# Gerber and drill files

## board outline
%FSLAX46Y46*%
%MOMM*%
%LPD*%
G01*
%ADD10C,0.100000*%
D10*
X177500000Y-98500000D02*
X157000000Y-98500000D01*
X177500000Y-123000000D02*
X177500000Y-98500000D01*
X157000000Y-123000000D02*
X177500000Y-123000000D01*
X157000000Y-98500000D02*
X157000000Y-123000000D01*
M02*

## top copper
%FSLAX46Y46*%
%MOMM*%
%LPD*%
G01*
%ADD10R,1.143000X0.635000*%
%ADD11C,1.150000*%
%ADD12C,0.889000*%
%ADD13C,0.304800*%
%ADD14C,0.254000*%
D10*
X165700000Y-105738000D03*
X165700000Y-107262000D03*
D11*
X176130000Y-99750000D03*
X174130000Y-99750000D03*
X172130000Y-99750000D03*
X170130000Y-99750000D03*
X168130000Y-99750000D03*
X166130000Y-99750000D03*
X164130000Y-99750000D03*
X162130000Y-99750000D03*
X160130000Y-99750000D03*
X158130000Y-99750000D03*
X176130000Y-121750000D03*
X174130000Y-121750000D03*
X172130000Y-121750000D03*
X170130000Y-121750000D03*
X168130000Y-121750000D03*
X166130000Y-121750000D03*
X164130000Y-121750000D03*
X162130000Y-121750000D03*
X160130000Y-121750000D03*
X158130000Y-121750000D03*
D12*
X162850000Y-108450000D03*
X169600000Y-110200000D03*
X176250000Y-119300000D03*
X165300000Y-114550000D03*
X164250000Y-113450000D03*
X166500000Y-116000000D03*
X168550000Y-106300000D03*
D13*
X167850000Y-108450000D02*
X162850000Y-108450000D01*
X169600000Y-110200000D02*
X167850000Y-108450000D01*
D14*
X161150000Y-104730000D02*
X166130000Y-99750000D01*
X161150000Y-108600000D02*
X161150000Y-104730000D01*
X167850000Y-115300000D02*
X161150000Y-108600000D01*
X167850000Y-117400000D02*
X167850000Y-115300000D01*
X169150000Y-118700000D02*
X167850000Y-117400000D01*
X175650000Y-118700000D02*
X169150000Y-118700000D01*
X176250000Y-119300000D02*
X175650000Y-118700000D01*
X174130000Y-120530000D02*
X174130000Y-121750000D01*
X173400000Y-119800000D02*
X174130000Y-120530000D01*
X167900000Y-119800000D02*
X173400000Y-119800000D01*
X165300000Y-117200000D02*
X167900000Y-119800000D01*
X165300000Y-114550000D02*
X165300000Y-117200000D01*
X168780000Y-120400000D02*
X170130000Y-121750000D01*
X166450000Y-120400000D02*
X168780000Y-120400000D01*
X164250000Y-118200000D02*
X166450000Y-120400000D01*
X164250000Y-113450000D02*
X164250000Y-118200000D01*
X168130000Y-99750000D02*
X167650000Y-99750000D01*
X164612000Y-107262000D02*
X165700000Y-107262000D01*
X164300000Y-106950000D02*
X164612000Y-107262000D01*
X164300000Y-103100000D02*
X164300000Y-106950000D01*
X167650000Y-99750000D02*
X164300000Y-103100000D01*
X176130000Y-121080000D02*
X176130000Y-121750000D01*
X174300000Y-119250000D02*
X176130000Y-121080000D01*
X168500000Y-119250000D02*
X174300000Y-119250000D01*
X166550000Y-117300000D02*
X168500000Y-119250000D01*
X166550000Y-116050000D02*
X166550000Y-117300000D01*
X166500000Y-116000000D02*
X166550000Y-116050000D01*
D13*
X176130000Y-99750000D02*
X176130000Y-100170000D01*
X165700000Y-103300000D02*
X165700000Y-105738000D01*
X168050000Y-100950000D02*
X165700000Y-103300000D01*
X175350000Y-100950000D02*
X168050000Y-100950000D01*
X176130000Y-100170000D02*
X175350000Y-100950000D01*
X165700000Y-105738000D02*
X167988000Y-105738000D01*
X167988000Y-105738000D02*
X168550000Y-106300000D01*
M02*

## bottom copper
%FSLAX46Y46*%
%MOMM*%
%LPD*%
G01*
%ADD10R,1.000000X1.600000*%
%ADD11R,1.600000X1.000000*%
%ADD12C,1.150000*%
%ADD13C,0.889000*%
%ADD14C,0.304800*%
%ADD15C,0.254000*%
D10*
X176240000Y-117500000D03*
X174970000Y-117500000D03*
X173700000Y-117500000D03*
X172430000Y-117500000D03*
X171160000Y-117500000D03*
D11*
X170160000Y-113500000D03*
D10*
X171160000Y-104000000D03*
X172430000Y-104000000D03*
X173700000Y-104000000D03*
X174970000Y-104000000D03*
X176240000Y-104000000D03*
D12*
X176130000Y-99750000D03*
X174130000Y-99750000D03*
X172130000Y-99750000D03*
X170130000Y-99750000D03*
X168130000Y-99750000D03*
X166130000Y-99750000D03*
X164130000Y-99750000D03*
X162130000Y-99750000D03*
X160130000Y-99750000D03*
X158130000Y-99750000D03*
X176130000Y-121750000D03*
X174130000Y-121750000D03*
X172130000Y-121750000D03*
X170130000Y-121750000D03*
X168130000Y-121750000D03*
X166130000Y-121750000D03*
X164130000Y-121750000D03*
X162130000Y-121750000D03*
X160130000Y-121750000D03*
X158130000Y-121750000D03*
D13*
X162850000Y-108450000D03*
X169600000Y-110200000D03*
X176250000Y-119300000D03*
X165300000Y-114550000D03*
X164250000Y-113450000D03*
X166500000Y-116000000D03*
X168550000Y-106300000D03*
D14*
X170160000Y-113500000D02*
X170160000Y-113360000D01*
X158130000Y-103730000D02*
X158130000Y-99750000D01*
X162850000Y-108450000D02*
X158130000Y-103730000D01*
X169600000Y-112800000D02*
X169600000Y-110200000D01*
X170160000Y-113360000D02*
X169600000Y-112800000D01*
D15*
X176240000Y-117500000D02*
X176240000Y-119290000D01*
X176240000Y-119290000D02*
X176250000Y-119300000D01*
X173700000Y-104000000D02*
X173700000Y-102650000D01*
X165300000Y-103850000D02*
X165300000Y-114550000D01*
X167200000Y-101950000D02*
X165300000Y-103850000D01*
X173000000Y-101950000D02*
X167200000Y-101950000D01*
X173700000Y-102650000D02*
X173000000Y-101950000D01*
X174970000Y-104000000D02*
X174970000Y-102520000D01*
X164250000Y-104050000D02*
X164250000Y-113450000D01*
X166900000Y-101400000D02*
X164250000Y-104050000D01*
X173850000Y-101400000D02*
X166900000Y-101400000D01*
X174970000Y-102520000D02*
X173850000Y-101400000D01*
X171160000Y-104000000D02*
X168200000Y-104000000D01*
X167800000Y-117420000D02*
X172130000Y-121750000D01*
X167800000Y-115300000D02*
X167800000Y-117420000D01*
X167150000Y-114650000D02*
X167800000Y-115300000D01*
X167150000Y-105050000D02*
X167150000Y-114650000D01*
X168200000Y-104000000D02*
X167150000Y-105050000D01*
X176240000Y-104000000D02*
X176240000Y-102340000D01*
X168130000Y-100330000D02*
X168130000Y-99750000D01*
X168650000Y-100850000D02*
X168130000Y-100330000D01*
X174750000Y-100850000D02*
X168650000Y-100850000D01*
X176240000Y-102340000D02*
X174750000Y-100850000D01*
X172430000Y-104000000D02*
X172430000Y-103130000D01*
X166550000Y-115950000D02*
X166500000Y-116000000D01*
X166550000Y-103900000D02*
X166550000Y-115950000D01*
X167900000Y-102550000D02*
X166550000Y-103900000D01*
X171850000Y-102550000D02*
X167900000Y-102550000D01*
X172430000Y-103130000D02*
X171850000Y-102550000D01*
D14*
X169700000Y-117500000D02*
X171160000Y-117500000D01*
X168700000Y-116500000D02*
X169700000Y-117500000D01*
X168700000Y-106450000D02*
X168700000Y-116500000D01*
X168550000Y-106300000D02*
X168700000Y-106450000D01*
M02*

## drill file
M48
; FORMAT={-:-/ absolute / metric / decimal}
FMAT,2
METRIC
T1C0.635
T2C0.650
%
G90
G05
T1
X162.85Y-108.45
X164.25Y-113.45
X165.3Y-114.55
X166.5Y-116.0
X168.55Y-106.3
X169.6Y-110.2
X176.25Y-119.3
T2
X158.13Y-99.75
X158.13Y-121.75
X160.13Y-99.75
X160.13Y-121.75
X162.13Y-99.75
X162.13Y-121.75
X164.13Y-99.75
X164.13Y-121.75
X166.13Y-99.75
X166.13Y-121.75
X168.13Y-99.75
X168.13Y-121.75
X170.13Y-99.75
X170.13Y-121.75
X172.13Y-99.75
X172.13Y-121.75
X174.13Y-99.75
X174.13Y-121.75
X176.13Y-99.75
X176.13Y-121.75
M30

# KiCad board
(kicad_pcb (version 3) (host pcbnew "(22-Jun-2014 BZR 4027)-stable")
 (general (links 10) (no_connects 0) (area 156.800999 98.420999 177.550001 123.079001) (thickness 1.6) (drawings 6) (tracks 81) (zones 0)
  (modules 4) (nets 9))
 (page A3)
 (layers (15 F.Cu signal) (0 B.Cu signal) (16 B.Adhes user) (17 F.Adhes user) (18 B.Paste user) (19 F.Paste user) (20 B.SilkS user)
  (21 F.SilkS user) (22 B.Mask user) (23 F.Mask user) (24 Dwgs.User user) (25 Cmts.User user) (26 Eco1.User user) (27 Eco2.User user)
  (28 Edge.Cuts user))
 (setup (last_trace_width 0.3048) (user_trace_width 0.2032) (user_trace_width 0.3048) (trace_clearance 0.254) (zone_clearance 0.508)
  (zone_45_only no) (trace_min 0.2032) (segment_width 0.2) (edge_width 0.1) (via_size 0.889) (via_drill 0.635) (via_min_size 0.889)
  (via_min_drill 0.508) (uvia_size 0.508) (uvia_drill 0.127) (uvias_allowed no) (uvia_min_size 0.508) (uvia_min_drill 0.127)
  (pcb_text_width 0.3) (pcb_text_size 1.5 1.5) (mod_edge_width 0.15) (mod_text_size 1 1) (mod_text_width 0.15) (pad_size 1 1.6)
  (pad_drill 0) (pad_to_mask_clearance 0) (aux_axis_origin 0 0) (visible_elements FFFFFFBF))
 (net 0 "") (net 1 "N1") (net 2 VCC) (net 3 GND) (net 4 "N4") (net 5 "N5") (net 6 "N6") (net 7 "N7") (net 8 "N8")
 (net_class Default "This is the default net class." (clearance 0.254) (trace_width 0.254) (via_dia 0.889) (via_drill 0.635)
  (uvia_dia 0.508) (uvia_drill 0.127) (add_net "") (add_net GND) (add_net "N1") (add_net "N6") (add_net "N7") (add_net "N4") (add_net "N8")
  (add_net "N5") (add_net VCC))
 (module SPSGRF (layer B.Cu) (at 173.7 110.75 90) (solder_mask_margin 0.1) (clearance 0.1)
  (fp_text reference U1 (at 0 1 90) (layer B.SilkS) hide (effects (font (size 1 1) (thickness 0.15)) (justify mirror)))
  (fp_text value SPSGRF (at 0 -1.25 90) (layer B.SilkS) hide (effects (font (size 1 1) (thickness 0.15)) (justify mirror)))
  (pad 1 smd rect (at -6.75 2.54 90) (size 1.6 1) (layers B.Cu B.Paste B.Mask) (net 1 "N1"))
  (pad 2 smd rect (at -6.75 1.27 90) (size 1.6 1) (layers B.Cu B.Paste B.Mask))
  (pad 3 smd rect (at -6.75 0 90) (size 1.6 1) (layers B.Cu B.Paste B.Mask))
  (pad 4 smd rect (at -6.75 -1.27 90) (size 1.6 1) (layers B.Cu B.Paste B.Mask))
  (pad 5 smd rect (at -6.75 -2.54 90) (size 1.6 1) (layers B.Cu B.Paste B.Mask) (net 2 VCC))
  (pad 6 smd rect (at -2.75 -3.54 90) (size 1 1.6) (layers B.Cu B.Paste B.Mask) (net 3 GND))
  (pad 7 smd rect (at 6.75 -2.54 90) (size 1.6 1) (layers B.Cu B.Paste B.Mask) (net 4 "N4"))
  (pad 8 smd rect (at 6.75 -1.27 90) (size 1.6 1) (layers B.Cu B.Paste B.Mask) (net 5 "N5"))
  (pad 9 smd rect (at 6.75 0 90) (size 1.6 1) (layers B.Cu B.Paste B.Mask) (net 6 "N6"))
  (pad 10 smd rect (at 6.75 1.27 90) (size 1.6 1) (layers B.Cu B.Paste B.Mask) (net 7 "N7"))
  (pad 11 smd rect (at 6.75 2.54 90) (size 1.6 1) (layers B.Cu B.Paste B.Mask) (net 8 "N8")))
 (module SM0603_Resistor (layer F.Cu) (at 165.7 106.5 270)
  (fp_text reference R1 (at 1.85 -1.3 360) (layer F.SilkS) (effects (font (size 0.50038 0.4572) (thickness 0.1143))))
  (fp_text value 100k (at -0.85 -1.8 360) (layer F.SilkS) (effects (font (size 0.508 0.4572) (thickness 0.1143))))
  (pad 1 smd rect (at -0.762 0 270) (size 0.635 1.143) (layers F.Cu F.Paste F.Mask) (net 2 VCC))
  (pad 2 smd rect (at 0.762 0 270) (size 0.635 1.143) (layers F.Cu F.Paste F.Mask) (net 8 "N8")))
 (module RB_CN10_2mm (layer F.Cu) (at 167.13 110.75)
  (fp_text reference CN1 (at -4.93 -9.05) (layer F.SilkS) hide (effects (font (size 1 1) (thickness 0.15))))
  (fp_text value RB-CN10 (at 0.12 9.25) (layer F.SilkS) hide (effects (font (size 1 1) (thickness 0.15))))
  (pad 1 thru_hole circle (at 9 -11) (size 1.15 1.15) (drill 0.65) (layers *.Cu *.Mask F.SilkS) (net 2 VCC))
  (pad 2 thru_hole circle (at 7 -11) (size 1.15 1.15) (drill 0.65) (layers *.Cu *.Mask F.SilkS))
  (pad 3 thru_hole circle (at 5 -11) (size 1.15 1.15) (drill 0.65) (layers *.Cu *.Mask F.SilkS))
  (pad 4 thru_hole circle (at 3 -11) (size 1.15 1.15) (drill 0.65) (layers *.Cu *.Mask F.SilkS))
  (pad 5 thru_hole circle (at 1 -11) (size 1.15 1.15) (drill 0.65) (layers *.Cu *.Mask F.SilkS) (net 8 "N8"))
  (pad 6 thru_hole circle (at -1 -11) (size 1.15 1.15) (drill 0.65) (layers *.Cu *.Mask F.SilkS) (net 1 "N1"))
  (pad 7 thru_hole circle (at -3 -11) (size 1.15 1.15) (drill 0.65) (layers *.Cu *.Mask F.SilkS))
  (pad 8 thru_hole circle (at -5 -11) (size 1.15 1.15) (drill 0.65) (layers *.Cu *.Mask F.SilkS))
  (pad 9 thru_hole circle (at -7 -11) (size 1.15 1.15) (drill 0.65) (layers *.Cu *.Mask F.SilkS))
  (pad 10 thru_hole circle (at -9 -11) (size 1.15 1.15) (drill 0.65) (layers *.Cu *.Mask F.SilkS) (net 3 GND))
  (pad 11 thru_hole circle (at 9 11) (size 1.15 1.15) (drill 0.65) (layers *.Cu *.Mask F.SilkS) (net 5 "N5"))
  (pad 12 thru_hole circle (at 7 11) (size 1.15 1.15) (drill 0.65) (layers *.Cu *.Mask F.SilkS) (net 6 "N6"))
  (pad 13 thru_hole circle (at 5 11) (size 1.15 1.15) (drill 0.65) (layers *.Cu *.Mask F.SilkS) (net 4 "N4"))
  (pad 14 thru_hole circle (at 3 11) (size 1.15 1.15) (drill 0.65) (layers *.Cu *.Mask F.SilkS) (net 7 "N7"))
  (pad 15 thru_hole circle (at 1 11) (size 1.15 1.15) (drill 0.65) (layers *.Cu *.Mask F.SilkS))
  (pad 16 thru_hole circle (at -1 11) (size 1.15 1.15) (drill 0.65) (layers *.Cu *.Mask F.SilkS))
  (pad 17 thru_hole circle (at -3 11) (size 1.15 1.15) (drill 0.65) (layers *.Cu *.Mask F.SilkS))
  (pad 18 thru_hole circle (at -5 11) (size 1.15 1.15) (drill 0.65) (layers *.Cu *.Mask F.SilkS))
  (pad 19 thru_hole circle (at -7 11) (size 1.15 1.15) (drill 0.65) (layers *.Cu *.Mask F.SilkS))
  (pad 20 thru_hole circle (at -9 11) (size 1.15 1.15) (drill 0.65) (layers *.Cu *.Mask F.SilkS)))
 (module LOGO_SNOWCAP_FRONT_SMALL (layer F.Cu) (at 172 110.95 270)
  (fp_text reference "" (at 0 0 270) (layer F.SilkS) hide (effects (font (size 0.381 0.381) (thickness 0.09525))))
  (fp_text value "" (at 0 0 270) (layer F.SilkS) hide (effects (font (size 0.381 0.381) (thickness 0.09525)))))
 (gr_line (start 177.5 98.5) (end 157 98.5) (angle 90) (layer Edge.Cuts) (width 0.1))
 (gr_line (start 177.5 123) (end 177.5 98.5) (angle 90) (layer Edge.Cuts) (width 0.1))
 (gr_line (start 157 123) (end 177.5 123) (angle 90) (layer Edge.Cuts) (width 0.1))
 (gr_line (start 157 98.5) (end 157 123) (angle 90) (layer Edge.Cuts) (width 0.1))
 (segment (start 170.16 113.5) (end 170.16 113.36) (width 0.3048) (layer B.Cu) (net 3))
 (segment (start 158.13 103.73) (end 158.13 99.75) (width 0.3048) (layer B.Cu) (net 3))
 (segment (start 162.85 108.45) (end 158.13 103.73) (width 0.3048) (layer B.Cu) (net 3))
 (via (at 162.85 108.45) (size 0.889) (layers F.Cu B.Cu) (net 3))
 (segment (start 167.85 108.45) (end 162.85 108.45) (width 0.3048) (layer F.Cu) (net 3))
 (segment (start 169.6 110.2) (end 167.85 108.45) (width 0.3048) (layer F.Cu) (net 3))
 (via (at 169.6 110.2) (size 0.889) (layers F.Cu B.Cu) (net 3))
 (segment (start 169.6 112.8) (end 169.6 110.2) (width 0.3048) (layer B.Cu) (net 3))
 (segment (start 170.16 113.36) (end 169.6 112.8) (width 0.3048) (layer B.Cu) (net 3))
 (segment (start 176.24 117.5) (end 176.24 119.29) (width 0.254) (layer B.Cu) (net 1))
 (segment (start 161.15 104.73) (end 166.13 99.75) (width 0.254) (layer F.Cu) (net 1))
 (segment (start 161.15 108.6) (end 161.15 104.73) (width 0.254) (layer F.Cu) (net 1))
 (segment (start 167.85 115.3) (end 161.15 108.6) (width 0.254) (layer F.Cu) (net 1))
 (segment (start 167.85 117.4) (end 167.85 115.3) (width 0.254) (layer F.Cu) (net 1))
 (segment (start 169.15 118.7) (end 167.85 117.4) (width 0.254) (layer F.Cu) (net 1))
 (segment (start 175.65 118.7) (end 169.15 118.7) (width 0.254) (layer F.Cu) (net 1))
 (segment (start 176.25 119.3) (end 175.65 118.7) (width 0.254) (layer F.Cu) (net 1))
 (via (at 176.25 119.3) (size 0.889) (layers F.Cu B.Cu) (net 1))
 (segment (start 176.24 119.29) (end 176.25 119.3) (width 0.254) (layer B.Cu) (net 1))
 (segment (start 173.7 104) (end 173.7 102.65) (width 0.254) (layer B.Cu) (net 6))
 (segment (start 174.13 120.53) (end 174.13 121.75) (width 0.254) (layer F.Cu) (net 6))
 (segment (start 173.4 119.8) (end 174.13 120.53) (width 0.254) (layer F.Cu) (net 6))
 (segment (start 167.9 119.8) (end 173.4 119.8) (width 0.254) (layer F.Cu) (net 6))
 (segment (start 165.3 117.2) (end 167.9 119.8) (width 0.254) (layer F.Cu) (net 6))
 (segment (start 165.3 114.55) (end 165.3 117.2) (width 0.254) (layer F.Cu) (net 6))
 (via (at 165.3 114.55) (size 0.889) (layers F.Cu B.Cu) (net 6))
 (segment (start 165.3 103.85) (end 165.3 114.55) (width 0.254) (layer B.Cu) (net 6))
 (segment (start 167.2 101.95) (end 165.3 103.85) (width 0.254) (layer B.Cu) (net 6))
 (segment (start 173 101.95) (end 167.2 101.95) (width 0.254) (layer B.Cu) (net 6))
 (segment (start 173.7 102.65) (end 173 101.95) (width 0.254) (layer B.Cu) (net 6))
 (segment (start 174.97 104) (end 174.97 102.52) (width 0.254) (layer B.Cu) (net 7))
 (segment (start 168.78 120.4) (end 170.13 121.75) (width 0.254) (layer F.Cu) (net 7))
 (segment (start 166.45 120.4) (end 168.78 120.4) (width 0.254) (layer F.Cu) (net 7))
 (segment (start 164.25 118.2) (end 166.45 120.4) (width 0.254) (layer F.Cu) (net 7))
 (segment (start 164.25 113.45) (end 164.25 118.2) (width 0.254) (layer F.Cu) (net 7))
 (via (at 164.25 113.45) (size 0.889) (layers F.Cu B.Cu) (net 7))
 (segment (start 164.25 104.05) (end 164.25 113.45) (width 0.254) (layer B.Cu) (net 7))
 (segment (start 166.9 101.4) (end 164.25 104.05) (width 0.254) (layer B.Cu) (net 7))
 (segment (start 173.85 101.4) (end 166.9 101.4) (width 0.254) (layer B.Cu) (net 7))
 (segment (start 174.97 102.52) (end 173.85 101.4) (width 0.254) (layer B.Cu) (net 7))
 (segment (start 171.16 104) (end 168.2 104) (width 0.254) (layer B.Cu) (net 4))
 (segment (start 167.8 117.42) (end 172.13 121.75) (width 0.254) (layer B.Cu) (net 4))
 (segment (start 167.8 115.3) (end 167.8 117.42) (width 0.254) (layer B.Cu) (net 4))
 (segment (start 167.15 114.65) (end 167.8 115.3) (width 0.254) (layer B.Cu) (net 4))
 (segment (start 167.15 105.05) (end 167.15 114.65) (width 0.254) (layer B.Cu) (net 4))
 (segment (start 168.2 104) (end 167.15 105.05) (width 0.254) (layer B.Cu) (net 4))
 (segment (start 168.13 99.75) (end 167.65 99.75) (width 0.254) (layer F.Cu) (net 8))
 (segment (start 164.612 107.262) (end 165.7 107.262) (width 0.254) (layer F.Cu) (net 8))
 (segment (start 164.3 106.95) (end 164.612 107.262) (width 0.254) (layer F.Cu) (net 8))
 (segment (start 164.3 103.1) (end 164.3 106.95) (width 0.254) (layer F.Cu) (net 8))
 (segment (start 167.65 99.75) (end 164.3 103.1) (width 0.254) (layer F.Cu) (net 8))
 (segment (start 176.24 104) (end 176.24 102.34) (width 0.254) (layer B.Cu) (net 8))
 (segment (start 168.13 100.33) (end 168.13 99.75) (width 0.254) (layer B.Cu) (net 8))
 (segment (start 168.65 100.85) (end 168.13 100.33) (width 0.254) (layer B.Cu) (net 8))
 (segment (start 174.75 100.85) (end 168.65 100.85) (width 0.254) (layer B.Cu) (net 8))
 (segment (start 176.24 102.34) (end 174.75 100.85) (width 0.254) (layer B.Cu) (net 8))
 (segment (start 172.43 104) (end 172.43 103.13) (width 0.254) (layer B.Cu) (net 5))
 (segment (start 176.13 121.08) (end 176.13 121.75) (width 0.254) (layer F.Cu) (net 5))
 (segment (start 174.3 119.25) (end 176.13 121.08) (width 0.254) (layer F.Cu) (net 5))
 (segment (start 168.5 119.25) (end 174.3 119.25) (width 0.254) (layer F.Cu) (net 5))
 (segment (start 166.55 117.3) (end 168.5 119.25) (width 0.254) (layer F.Cu) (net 5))
 (segment (start 166.55 116.05) (end 166.55 117.3) (width 0.254) (layer F.Cu) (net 5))
 (segment (start 166.5 116) (end 166.55 116.05) (width 0.254) (layer F.Cu) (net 5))
 (via (at 166.5 116) (size 0.889) (layers F.Cu B.Cu) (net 5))
 (segment (start 166.55 115.95) (end 166.5 116) (width 0.254) (layer B.Cu) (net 5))
 (segment (start 166.55 103.9) (end 166.55 115.95) (width 0.254) (layer B.Cu) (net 5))
 (segment (start 167.9 102.55) (end 166.55 103.9) (width 0.254) (layer B.Cu) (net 5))
 (segment (start 171.85 102.55) (end 167.9 102.55) (width 0.254) (layer B.Cu) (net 5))
 (segment (start 172.43 103.13) (end 171.85 102.55) (width 0.254) (layer B.Cu) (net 5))
 (segment (start 176.13 99.75) (end 176.13 100.17) (width 0.3048) (layer F.Cu) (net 2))
 (segment (start 165.7 103.3) (end 165.7 105.738) (width 0.3048) (layer F.Cu) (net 2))
 (segment (start 168.05 100.95) (end 165.7 103.3) (width 0.3048) (layer F.Cu) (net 2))
 (segment (start 175.35 100.95) (end 168.05 100.95) (width 0.3048) (layer F.Cu) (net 2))
 (segment (start 176.13 100.17) (end 175.35 100.95) (width 0.3048) (layer F.Cu) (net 2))
 (segment (start 165.7 105.738) (end 167.988 105.738) (width 0.3048) (layer F.Cu) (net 2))
 (segment (start 169.7 117.5) (end 171.16 117.5) (width 0.3048) (layer B.Cu) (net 2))
 (segment (start 168.7 116.5) (end 169.7 117.5) (width 0.3048) (layer B.Cu) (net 2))
 (segment (start 168.7 106.45) (end 168.7 116.5) (width 0.3048) (layer B.Cu) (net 2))
 (segment (start 168.55 106.3) (end 168.7 106.45) (width 0.3048) (layer B.Cu) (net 2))
 (via (at 168.55 106.3) (size 0.889) (layers F.Cu B.Cu) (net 2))
 (segment (start 167.988 105.738) (end 168.55 106.3) (width 0.3048) (layer F.Cu) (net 2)))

